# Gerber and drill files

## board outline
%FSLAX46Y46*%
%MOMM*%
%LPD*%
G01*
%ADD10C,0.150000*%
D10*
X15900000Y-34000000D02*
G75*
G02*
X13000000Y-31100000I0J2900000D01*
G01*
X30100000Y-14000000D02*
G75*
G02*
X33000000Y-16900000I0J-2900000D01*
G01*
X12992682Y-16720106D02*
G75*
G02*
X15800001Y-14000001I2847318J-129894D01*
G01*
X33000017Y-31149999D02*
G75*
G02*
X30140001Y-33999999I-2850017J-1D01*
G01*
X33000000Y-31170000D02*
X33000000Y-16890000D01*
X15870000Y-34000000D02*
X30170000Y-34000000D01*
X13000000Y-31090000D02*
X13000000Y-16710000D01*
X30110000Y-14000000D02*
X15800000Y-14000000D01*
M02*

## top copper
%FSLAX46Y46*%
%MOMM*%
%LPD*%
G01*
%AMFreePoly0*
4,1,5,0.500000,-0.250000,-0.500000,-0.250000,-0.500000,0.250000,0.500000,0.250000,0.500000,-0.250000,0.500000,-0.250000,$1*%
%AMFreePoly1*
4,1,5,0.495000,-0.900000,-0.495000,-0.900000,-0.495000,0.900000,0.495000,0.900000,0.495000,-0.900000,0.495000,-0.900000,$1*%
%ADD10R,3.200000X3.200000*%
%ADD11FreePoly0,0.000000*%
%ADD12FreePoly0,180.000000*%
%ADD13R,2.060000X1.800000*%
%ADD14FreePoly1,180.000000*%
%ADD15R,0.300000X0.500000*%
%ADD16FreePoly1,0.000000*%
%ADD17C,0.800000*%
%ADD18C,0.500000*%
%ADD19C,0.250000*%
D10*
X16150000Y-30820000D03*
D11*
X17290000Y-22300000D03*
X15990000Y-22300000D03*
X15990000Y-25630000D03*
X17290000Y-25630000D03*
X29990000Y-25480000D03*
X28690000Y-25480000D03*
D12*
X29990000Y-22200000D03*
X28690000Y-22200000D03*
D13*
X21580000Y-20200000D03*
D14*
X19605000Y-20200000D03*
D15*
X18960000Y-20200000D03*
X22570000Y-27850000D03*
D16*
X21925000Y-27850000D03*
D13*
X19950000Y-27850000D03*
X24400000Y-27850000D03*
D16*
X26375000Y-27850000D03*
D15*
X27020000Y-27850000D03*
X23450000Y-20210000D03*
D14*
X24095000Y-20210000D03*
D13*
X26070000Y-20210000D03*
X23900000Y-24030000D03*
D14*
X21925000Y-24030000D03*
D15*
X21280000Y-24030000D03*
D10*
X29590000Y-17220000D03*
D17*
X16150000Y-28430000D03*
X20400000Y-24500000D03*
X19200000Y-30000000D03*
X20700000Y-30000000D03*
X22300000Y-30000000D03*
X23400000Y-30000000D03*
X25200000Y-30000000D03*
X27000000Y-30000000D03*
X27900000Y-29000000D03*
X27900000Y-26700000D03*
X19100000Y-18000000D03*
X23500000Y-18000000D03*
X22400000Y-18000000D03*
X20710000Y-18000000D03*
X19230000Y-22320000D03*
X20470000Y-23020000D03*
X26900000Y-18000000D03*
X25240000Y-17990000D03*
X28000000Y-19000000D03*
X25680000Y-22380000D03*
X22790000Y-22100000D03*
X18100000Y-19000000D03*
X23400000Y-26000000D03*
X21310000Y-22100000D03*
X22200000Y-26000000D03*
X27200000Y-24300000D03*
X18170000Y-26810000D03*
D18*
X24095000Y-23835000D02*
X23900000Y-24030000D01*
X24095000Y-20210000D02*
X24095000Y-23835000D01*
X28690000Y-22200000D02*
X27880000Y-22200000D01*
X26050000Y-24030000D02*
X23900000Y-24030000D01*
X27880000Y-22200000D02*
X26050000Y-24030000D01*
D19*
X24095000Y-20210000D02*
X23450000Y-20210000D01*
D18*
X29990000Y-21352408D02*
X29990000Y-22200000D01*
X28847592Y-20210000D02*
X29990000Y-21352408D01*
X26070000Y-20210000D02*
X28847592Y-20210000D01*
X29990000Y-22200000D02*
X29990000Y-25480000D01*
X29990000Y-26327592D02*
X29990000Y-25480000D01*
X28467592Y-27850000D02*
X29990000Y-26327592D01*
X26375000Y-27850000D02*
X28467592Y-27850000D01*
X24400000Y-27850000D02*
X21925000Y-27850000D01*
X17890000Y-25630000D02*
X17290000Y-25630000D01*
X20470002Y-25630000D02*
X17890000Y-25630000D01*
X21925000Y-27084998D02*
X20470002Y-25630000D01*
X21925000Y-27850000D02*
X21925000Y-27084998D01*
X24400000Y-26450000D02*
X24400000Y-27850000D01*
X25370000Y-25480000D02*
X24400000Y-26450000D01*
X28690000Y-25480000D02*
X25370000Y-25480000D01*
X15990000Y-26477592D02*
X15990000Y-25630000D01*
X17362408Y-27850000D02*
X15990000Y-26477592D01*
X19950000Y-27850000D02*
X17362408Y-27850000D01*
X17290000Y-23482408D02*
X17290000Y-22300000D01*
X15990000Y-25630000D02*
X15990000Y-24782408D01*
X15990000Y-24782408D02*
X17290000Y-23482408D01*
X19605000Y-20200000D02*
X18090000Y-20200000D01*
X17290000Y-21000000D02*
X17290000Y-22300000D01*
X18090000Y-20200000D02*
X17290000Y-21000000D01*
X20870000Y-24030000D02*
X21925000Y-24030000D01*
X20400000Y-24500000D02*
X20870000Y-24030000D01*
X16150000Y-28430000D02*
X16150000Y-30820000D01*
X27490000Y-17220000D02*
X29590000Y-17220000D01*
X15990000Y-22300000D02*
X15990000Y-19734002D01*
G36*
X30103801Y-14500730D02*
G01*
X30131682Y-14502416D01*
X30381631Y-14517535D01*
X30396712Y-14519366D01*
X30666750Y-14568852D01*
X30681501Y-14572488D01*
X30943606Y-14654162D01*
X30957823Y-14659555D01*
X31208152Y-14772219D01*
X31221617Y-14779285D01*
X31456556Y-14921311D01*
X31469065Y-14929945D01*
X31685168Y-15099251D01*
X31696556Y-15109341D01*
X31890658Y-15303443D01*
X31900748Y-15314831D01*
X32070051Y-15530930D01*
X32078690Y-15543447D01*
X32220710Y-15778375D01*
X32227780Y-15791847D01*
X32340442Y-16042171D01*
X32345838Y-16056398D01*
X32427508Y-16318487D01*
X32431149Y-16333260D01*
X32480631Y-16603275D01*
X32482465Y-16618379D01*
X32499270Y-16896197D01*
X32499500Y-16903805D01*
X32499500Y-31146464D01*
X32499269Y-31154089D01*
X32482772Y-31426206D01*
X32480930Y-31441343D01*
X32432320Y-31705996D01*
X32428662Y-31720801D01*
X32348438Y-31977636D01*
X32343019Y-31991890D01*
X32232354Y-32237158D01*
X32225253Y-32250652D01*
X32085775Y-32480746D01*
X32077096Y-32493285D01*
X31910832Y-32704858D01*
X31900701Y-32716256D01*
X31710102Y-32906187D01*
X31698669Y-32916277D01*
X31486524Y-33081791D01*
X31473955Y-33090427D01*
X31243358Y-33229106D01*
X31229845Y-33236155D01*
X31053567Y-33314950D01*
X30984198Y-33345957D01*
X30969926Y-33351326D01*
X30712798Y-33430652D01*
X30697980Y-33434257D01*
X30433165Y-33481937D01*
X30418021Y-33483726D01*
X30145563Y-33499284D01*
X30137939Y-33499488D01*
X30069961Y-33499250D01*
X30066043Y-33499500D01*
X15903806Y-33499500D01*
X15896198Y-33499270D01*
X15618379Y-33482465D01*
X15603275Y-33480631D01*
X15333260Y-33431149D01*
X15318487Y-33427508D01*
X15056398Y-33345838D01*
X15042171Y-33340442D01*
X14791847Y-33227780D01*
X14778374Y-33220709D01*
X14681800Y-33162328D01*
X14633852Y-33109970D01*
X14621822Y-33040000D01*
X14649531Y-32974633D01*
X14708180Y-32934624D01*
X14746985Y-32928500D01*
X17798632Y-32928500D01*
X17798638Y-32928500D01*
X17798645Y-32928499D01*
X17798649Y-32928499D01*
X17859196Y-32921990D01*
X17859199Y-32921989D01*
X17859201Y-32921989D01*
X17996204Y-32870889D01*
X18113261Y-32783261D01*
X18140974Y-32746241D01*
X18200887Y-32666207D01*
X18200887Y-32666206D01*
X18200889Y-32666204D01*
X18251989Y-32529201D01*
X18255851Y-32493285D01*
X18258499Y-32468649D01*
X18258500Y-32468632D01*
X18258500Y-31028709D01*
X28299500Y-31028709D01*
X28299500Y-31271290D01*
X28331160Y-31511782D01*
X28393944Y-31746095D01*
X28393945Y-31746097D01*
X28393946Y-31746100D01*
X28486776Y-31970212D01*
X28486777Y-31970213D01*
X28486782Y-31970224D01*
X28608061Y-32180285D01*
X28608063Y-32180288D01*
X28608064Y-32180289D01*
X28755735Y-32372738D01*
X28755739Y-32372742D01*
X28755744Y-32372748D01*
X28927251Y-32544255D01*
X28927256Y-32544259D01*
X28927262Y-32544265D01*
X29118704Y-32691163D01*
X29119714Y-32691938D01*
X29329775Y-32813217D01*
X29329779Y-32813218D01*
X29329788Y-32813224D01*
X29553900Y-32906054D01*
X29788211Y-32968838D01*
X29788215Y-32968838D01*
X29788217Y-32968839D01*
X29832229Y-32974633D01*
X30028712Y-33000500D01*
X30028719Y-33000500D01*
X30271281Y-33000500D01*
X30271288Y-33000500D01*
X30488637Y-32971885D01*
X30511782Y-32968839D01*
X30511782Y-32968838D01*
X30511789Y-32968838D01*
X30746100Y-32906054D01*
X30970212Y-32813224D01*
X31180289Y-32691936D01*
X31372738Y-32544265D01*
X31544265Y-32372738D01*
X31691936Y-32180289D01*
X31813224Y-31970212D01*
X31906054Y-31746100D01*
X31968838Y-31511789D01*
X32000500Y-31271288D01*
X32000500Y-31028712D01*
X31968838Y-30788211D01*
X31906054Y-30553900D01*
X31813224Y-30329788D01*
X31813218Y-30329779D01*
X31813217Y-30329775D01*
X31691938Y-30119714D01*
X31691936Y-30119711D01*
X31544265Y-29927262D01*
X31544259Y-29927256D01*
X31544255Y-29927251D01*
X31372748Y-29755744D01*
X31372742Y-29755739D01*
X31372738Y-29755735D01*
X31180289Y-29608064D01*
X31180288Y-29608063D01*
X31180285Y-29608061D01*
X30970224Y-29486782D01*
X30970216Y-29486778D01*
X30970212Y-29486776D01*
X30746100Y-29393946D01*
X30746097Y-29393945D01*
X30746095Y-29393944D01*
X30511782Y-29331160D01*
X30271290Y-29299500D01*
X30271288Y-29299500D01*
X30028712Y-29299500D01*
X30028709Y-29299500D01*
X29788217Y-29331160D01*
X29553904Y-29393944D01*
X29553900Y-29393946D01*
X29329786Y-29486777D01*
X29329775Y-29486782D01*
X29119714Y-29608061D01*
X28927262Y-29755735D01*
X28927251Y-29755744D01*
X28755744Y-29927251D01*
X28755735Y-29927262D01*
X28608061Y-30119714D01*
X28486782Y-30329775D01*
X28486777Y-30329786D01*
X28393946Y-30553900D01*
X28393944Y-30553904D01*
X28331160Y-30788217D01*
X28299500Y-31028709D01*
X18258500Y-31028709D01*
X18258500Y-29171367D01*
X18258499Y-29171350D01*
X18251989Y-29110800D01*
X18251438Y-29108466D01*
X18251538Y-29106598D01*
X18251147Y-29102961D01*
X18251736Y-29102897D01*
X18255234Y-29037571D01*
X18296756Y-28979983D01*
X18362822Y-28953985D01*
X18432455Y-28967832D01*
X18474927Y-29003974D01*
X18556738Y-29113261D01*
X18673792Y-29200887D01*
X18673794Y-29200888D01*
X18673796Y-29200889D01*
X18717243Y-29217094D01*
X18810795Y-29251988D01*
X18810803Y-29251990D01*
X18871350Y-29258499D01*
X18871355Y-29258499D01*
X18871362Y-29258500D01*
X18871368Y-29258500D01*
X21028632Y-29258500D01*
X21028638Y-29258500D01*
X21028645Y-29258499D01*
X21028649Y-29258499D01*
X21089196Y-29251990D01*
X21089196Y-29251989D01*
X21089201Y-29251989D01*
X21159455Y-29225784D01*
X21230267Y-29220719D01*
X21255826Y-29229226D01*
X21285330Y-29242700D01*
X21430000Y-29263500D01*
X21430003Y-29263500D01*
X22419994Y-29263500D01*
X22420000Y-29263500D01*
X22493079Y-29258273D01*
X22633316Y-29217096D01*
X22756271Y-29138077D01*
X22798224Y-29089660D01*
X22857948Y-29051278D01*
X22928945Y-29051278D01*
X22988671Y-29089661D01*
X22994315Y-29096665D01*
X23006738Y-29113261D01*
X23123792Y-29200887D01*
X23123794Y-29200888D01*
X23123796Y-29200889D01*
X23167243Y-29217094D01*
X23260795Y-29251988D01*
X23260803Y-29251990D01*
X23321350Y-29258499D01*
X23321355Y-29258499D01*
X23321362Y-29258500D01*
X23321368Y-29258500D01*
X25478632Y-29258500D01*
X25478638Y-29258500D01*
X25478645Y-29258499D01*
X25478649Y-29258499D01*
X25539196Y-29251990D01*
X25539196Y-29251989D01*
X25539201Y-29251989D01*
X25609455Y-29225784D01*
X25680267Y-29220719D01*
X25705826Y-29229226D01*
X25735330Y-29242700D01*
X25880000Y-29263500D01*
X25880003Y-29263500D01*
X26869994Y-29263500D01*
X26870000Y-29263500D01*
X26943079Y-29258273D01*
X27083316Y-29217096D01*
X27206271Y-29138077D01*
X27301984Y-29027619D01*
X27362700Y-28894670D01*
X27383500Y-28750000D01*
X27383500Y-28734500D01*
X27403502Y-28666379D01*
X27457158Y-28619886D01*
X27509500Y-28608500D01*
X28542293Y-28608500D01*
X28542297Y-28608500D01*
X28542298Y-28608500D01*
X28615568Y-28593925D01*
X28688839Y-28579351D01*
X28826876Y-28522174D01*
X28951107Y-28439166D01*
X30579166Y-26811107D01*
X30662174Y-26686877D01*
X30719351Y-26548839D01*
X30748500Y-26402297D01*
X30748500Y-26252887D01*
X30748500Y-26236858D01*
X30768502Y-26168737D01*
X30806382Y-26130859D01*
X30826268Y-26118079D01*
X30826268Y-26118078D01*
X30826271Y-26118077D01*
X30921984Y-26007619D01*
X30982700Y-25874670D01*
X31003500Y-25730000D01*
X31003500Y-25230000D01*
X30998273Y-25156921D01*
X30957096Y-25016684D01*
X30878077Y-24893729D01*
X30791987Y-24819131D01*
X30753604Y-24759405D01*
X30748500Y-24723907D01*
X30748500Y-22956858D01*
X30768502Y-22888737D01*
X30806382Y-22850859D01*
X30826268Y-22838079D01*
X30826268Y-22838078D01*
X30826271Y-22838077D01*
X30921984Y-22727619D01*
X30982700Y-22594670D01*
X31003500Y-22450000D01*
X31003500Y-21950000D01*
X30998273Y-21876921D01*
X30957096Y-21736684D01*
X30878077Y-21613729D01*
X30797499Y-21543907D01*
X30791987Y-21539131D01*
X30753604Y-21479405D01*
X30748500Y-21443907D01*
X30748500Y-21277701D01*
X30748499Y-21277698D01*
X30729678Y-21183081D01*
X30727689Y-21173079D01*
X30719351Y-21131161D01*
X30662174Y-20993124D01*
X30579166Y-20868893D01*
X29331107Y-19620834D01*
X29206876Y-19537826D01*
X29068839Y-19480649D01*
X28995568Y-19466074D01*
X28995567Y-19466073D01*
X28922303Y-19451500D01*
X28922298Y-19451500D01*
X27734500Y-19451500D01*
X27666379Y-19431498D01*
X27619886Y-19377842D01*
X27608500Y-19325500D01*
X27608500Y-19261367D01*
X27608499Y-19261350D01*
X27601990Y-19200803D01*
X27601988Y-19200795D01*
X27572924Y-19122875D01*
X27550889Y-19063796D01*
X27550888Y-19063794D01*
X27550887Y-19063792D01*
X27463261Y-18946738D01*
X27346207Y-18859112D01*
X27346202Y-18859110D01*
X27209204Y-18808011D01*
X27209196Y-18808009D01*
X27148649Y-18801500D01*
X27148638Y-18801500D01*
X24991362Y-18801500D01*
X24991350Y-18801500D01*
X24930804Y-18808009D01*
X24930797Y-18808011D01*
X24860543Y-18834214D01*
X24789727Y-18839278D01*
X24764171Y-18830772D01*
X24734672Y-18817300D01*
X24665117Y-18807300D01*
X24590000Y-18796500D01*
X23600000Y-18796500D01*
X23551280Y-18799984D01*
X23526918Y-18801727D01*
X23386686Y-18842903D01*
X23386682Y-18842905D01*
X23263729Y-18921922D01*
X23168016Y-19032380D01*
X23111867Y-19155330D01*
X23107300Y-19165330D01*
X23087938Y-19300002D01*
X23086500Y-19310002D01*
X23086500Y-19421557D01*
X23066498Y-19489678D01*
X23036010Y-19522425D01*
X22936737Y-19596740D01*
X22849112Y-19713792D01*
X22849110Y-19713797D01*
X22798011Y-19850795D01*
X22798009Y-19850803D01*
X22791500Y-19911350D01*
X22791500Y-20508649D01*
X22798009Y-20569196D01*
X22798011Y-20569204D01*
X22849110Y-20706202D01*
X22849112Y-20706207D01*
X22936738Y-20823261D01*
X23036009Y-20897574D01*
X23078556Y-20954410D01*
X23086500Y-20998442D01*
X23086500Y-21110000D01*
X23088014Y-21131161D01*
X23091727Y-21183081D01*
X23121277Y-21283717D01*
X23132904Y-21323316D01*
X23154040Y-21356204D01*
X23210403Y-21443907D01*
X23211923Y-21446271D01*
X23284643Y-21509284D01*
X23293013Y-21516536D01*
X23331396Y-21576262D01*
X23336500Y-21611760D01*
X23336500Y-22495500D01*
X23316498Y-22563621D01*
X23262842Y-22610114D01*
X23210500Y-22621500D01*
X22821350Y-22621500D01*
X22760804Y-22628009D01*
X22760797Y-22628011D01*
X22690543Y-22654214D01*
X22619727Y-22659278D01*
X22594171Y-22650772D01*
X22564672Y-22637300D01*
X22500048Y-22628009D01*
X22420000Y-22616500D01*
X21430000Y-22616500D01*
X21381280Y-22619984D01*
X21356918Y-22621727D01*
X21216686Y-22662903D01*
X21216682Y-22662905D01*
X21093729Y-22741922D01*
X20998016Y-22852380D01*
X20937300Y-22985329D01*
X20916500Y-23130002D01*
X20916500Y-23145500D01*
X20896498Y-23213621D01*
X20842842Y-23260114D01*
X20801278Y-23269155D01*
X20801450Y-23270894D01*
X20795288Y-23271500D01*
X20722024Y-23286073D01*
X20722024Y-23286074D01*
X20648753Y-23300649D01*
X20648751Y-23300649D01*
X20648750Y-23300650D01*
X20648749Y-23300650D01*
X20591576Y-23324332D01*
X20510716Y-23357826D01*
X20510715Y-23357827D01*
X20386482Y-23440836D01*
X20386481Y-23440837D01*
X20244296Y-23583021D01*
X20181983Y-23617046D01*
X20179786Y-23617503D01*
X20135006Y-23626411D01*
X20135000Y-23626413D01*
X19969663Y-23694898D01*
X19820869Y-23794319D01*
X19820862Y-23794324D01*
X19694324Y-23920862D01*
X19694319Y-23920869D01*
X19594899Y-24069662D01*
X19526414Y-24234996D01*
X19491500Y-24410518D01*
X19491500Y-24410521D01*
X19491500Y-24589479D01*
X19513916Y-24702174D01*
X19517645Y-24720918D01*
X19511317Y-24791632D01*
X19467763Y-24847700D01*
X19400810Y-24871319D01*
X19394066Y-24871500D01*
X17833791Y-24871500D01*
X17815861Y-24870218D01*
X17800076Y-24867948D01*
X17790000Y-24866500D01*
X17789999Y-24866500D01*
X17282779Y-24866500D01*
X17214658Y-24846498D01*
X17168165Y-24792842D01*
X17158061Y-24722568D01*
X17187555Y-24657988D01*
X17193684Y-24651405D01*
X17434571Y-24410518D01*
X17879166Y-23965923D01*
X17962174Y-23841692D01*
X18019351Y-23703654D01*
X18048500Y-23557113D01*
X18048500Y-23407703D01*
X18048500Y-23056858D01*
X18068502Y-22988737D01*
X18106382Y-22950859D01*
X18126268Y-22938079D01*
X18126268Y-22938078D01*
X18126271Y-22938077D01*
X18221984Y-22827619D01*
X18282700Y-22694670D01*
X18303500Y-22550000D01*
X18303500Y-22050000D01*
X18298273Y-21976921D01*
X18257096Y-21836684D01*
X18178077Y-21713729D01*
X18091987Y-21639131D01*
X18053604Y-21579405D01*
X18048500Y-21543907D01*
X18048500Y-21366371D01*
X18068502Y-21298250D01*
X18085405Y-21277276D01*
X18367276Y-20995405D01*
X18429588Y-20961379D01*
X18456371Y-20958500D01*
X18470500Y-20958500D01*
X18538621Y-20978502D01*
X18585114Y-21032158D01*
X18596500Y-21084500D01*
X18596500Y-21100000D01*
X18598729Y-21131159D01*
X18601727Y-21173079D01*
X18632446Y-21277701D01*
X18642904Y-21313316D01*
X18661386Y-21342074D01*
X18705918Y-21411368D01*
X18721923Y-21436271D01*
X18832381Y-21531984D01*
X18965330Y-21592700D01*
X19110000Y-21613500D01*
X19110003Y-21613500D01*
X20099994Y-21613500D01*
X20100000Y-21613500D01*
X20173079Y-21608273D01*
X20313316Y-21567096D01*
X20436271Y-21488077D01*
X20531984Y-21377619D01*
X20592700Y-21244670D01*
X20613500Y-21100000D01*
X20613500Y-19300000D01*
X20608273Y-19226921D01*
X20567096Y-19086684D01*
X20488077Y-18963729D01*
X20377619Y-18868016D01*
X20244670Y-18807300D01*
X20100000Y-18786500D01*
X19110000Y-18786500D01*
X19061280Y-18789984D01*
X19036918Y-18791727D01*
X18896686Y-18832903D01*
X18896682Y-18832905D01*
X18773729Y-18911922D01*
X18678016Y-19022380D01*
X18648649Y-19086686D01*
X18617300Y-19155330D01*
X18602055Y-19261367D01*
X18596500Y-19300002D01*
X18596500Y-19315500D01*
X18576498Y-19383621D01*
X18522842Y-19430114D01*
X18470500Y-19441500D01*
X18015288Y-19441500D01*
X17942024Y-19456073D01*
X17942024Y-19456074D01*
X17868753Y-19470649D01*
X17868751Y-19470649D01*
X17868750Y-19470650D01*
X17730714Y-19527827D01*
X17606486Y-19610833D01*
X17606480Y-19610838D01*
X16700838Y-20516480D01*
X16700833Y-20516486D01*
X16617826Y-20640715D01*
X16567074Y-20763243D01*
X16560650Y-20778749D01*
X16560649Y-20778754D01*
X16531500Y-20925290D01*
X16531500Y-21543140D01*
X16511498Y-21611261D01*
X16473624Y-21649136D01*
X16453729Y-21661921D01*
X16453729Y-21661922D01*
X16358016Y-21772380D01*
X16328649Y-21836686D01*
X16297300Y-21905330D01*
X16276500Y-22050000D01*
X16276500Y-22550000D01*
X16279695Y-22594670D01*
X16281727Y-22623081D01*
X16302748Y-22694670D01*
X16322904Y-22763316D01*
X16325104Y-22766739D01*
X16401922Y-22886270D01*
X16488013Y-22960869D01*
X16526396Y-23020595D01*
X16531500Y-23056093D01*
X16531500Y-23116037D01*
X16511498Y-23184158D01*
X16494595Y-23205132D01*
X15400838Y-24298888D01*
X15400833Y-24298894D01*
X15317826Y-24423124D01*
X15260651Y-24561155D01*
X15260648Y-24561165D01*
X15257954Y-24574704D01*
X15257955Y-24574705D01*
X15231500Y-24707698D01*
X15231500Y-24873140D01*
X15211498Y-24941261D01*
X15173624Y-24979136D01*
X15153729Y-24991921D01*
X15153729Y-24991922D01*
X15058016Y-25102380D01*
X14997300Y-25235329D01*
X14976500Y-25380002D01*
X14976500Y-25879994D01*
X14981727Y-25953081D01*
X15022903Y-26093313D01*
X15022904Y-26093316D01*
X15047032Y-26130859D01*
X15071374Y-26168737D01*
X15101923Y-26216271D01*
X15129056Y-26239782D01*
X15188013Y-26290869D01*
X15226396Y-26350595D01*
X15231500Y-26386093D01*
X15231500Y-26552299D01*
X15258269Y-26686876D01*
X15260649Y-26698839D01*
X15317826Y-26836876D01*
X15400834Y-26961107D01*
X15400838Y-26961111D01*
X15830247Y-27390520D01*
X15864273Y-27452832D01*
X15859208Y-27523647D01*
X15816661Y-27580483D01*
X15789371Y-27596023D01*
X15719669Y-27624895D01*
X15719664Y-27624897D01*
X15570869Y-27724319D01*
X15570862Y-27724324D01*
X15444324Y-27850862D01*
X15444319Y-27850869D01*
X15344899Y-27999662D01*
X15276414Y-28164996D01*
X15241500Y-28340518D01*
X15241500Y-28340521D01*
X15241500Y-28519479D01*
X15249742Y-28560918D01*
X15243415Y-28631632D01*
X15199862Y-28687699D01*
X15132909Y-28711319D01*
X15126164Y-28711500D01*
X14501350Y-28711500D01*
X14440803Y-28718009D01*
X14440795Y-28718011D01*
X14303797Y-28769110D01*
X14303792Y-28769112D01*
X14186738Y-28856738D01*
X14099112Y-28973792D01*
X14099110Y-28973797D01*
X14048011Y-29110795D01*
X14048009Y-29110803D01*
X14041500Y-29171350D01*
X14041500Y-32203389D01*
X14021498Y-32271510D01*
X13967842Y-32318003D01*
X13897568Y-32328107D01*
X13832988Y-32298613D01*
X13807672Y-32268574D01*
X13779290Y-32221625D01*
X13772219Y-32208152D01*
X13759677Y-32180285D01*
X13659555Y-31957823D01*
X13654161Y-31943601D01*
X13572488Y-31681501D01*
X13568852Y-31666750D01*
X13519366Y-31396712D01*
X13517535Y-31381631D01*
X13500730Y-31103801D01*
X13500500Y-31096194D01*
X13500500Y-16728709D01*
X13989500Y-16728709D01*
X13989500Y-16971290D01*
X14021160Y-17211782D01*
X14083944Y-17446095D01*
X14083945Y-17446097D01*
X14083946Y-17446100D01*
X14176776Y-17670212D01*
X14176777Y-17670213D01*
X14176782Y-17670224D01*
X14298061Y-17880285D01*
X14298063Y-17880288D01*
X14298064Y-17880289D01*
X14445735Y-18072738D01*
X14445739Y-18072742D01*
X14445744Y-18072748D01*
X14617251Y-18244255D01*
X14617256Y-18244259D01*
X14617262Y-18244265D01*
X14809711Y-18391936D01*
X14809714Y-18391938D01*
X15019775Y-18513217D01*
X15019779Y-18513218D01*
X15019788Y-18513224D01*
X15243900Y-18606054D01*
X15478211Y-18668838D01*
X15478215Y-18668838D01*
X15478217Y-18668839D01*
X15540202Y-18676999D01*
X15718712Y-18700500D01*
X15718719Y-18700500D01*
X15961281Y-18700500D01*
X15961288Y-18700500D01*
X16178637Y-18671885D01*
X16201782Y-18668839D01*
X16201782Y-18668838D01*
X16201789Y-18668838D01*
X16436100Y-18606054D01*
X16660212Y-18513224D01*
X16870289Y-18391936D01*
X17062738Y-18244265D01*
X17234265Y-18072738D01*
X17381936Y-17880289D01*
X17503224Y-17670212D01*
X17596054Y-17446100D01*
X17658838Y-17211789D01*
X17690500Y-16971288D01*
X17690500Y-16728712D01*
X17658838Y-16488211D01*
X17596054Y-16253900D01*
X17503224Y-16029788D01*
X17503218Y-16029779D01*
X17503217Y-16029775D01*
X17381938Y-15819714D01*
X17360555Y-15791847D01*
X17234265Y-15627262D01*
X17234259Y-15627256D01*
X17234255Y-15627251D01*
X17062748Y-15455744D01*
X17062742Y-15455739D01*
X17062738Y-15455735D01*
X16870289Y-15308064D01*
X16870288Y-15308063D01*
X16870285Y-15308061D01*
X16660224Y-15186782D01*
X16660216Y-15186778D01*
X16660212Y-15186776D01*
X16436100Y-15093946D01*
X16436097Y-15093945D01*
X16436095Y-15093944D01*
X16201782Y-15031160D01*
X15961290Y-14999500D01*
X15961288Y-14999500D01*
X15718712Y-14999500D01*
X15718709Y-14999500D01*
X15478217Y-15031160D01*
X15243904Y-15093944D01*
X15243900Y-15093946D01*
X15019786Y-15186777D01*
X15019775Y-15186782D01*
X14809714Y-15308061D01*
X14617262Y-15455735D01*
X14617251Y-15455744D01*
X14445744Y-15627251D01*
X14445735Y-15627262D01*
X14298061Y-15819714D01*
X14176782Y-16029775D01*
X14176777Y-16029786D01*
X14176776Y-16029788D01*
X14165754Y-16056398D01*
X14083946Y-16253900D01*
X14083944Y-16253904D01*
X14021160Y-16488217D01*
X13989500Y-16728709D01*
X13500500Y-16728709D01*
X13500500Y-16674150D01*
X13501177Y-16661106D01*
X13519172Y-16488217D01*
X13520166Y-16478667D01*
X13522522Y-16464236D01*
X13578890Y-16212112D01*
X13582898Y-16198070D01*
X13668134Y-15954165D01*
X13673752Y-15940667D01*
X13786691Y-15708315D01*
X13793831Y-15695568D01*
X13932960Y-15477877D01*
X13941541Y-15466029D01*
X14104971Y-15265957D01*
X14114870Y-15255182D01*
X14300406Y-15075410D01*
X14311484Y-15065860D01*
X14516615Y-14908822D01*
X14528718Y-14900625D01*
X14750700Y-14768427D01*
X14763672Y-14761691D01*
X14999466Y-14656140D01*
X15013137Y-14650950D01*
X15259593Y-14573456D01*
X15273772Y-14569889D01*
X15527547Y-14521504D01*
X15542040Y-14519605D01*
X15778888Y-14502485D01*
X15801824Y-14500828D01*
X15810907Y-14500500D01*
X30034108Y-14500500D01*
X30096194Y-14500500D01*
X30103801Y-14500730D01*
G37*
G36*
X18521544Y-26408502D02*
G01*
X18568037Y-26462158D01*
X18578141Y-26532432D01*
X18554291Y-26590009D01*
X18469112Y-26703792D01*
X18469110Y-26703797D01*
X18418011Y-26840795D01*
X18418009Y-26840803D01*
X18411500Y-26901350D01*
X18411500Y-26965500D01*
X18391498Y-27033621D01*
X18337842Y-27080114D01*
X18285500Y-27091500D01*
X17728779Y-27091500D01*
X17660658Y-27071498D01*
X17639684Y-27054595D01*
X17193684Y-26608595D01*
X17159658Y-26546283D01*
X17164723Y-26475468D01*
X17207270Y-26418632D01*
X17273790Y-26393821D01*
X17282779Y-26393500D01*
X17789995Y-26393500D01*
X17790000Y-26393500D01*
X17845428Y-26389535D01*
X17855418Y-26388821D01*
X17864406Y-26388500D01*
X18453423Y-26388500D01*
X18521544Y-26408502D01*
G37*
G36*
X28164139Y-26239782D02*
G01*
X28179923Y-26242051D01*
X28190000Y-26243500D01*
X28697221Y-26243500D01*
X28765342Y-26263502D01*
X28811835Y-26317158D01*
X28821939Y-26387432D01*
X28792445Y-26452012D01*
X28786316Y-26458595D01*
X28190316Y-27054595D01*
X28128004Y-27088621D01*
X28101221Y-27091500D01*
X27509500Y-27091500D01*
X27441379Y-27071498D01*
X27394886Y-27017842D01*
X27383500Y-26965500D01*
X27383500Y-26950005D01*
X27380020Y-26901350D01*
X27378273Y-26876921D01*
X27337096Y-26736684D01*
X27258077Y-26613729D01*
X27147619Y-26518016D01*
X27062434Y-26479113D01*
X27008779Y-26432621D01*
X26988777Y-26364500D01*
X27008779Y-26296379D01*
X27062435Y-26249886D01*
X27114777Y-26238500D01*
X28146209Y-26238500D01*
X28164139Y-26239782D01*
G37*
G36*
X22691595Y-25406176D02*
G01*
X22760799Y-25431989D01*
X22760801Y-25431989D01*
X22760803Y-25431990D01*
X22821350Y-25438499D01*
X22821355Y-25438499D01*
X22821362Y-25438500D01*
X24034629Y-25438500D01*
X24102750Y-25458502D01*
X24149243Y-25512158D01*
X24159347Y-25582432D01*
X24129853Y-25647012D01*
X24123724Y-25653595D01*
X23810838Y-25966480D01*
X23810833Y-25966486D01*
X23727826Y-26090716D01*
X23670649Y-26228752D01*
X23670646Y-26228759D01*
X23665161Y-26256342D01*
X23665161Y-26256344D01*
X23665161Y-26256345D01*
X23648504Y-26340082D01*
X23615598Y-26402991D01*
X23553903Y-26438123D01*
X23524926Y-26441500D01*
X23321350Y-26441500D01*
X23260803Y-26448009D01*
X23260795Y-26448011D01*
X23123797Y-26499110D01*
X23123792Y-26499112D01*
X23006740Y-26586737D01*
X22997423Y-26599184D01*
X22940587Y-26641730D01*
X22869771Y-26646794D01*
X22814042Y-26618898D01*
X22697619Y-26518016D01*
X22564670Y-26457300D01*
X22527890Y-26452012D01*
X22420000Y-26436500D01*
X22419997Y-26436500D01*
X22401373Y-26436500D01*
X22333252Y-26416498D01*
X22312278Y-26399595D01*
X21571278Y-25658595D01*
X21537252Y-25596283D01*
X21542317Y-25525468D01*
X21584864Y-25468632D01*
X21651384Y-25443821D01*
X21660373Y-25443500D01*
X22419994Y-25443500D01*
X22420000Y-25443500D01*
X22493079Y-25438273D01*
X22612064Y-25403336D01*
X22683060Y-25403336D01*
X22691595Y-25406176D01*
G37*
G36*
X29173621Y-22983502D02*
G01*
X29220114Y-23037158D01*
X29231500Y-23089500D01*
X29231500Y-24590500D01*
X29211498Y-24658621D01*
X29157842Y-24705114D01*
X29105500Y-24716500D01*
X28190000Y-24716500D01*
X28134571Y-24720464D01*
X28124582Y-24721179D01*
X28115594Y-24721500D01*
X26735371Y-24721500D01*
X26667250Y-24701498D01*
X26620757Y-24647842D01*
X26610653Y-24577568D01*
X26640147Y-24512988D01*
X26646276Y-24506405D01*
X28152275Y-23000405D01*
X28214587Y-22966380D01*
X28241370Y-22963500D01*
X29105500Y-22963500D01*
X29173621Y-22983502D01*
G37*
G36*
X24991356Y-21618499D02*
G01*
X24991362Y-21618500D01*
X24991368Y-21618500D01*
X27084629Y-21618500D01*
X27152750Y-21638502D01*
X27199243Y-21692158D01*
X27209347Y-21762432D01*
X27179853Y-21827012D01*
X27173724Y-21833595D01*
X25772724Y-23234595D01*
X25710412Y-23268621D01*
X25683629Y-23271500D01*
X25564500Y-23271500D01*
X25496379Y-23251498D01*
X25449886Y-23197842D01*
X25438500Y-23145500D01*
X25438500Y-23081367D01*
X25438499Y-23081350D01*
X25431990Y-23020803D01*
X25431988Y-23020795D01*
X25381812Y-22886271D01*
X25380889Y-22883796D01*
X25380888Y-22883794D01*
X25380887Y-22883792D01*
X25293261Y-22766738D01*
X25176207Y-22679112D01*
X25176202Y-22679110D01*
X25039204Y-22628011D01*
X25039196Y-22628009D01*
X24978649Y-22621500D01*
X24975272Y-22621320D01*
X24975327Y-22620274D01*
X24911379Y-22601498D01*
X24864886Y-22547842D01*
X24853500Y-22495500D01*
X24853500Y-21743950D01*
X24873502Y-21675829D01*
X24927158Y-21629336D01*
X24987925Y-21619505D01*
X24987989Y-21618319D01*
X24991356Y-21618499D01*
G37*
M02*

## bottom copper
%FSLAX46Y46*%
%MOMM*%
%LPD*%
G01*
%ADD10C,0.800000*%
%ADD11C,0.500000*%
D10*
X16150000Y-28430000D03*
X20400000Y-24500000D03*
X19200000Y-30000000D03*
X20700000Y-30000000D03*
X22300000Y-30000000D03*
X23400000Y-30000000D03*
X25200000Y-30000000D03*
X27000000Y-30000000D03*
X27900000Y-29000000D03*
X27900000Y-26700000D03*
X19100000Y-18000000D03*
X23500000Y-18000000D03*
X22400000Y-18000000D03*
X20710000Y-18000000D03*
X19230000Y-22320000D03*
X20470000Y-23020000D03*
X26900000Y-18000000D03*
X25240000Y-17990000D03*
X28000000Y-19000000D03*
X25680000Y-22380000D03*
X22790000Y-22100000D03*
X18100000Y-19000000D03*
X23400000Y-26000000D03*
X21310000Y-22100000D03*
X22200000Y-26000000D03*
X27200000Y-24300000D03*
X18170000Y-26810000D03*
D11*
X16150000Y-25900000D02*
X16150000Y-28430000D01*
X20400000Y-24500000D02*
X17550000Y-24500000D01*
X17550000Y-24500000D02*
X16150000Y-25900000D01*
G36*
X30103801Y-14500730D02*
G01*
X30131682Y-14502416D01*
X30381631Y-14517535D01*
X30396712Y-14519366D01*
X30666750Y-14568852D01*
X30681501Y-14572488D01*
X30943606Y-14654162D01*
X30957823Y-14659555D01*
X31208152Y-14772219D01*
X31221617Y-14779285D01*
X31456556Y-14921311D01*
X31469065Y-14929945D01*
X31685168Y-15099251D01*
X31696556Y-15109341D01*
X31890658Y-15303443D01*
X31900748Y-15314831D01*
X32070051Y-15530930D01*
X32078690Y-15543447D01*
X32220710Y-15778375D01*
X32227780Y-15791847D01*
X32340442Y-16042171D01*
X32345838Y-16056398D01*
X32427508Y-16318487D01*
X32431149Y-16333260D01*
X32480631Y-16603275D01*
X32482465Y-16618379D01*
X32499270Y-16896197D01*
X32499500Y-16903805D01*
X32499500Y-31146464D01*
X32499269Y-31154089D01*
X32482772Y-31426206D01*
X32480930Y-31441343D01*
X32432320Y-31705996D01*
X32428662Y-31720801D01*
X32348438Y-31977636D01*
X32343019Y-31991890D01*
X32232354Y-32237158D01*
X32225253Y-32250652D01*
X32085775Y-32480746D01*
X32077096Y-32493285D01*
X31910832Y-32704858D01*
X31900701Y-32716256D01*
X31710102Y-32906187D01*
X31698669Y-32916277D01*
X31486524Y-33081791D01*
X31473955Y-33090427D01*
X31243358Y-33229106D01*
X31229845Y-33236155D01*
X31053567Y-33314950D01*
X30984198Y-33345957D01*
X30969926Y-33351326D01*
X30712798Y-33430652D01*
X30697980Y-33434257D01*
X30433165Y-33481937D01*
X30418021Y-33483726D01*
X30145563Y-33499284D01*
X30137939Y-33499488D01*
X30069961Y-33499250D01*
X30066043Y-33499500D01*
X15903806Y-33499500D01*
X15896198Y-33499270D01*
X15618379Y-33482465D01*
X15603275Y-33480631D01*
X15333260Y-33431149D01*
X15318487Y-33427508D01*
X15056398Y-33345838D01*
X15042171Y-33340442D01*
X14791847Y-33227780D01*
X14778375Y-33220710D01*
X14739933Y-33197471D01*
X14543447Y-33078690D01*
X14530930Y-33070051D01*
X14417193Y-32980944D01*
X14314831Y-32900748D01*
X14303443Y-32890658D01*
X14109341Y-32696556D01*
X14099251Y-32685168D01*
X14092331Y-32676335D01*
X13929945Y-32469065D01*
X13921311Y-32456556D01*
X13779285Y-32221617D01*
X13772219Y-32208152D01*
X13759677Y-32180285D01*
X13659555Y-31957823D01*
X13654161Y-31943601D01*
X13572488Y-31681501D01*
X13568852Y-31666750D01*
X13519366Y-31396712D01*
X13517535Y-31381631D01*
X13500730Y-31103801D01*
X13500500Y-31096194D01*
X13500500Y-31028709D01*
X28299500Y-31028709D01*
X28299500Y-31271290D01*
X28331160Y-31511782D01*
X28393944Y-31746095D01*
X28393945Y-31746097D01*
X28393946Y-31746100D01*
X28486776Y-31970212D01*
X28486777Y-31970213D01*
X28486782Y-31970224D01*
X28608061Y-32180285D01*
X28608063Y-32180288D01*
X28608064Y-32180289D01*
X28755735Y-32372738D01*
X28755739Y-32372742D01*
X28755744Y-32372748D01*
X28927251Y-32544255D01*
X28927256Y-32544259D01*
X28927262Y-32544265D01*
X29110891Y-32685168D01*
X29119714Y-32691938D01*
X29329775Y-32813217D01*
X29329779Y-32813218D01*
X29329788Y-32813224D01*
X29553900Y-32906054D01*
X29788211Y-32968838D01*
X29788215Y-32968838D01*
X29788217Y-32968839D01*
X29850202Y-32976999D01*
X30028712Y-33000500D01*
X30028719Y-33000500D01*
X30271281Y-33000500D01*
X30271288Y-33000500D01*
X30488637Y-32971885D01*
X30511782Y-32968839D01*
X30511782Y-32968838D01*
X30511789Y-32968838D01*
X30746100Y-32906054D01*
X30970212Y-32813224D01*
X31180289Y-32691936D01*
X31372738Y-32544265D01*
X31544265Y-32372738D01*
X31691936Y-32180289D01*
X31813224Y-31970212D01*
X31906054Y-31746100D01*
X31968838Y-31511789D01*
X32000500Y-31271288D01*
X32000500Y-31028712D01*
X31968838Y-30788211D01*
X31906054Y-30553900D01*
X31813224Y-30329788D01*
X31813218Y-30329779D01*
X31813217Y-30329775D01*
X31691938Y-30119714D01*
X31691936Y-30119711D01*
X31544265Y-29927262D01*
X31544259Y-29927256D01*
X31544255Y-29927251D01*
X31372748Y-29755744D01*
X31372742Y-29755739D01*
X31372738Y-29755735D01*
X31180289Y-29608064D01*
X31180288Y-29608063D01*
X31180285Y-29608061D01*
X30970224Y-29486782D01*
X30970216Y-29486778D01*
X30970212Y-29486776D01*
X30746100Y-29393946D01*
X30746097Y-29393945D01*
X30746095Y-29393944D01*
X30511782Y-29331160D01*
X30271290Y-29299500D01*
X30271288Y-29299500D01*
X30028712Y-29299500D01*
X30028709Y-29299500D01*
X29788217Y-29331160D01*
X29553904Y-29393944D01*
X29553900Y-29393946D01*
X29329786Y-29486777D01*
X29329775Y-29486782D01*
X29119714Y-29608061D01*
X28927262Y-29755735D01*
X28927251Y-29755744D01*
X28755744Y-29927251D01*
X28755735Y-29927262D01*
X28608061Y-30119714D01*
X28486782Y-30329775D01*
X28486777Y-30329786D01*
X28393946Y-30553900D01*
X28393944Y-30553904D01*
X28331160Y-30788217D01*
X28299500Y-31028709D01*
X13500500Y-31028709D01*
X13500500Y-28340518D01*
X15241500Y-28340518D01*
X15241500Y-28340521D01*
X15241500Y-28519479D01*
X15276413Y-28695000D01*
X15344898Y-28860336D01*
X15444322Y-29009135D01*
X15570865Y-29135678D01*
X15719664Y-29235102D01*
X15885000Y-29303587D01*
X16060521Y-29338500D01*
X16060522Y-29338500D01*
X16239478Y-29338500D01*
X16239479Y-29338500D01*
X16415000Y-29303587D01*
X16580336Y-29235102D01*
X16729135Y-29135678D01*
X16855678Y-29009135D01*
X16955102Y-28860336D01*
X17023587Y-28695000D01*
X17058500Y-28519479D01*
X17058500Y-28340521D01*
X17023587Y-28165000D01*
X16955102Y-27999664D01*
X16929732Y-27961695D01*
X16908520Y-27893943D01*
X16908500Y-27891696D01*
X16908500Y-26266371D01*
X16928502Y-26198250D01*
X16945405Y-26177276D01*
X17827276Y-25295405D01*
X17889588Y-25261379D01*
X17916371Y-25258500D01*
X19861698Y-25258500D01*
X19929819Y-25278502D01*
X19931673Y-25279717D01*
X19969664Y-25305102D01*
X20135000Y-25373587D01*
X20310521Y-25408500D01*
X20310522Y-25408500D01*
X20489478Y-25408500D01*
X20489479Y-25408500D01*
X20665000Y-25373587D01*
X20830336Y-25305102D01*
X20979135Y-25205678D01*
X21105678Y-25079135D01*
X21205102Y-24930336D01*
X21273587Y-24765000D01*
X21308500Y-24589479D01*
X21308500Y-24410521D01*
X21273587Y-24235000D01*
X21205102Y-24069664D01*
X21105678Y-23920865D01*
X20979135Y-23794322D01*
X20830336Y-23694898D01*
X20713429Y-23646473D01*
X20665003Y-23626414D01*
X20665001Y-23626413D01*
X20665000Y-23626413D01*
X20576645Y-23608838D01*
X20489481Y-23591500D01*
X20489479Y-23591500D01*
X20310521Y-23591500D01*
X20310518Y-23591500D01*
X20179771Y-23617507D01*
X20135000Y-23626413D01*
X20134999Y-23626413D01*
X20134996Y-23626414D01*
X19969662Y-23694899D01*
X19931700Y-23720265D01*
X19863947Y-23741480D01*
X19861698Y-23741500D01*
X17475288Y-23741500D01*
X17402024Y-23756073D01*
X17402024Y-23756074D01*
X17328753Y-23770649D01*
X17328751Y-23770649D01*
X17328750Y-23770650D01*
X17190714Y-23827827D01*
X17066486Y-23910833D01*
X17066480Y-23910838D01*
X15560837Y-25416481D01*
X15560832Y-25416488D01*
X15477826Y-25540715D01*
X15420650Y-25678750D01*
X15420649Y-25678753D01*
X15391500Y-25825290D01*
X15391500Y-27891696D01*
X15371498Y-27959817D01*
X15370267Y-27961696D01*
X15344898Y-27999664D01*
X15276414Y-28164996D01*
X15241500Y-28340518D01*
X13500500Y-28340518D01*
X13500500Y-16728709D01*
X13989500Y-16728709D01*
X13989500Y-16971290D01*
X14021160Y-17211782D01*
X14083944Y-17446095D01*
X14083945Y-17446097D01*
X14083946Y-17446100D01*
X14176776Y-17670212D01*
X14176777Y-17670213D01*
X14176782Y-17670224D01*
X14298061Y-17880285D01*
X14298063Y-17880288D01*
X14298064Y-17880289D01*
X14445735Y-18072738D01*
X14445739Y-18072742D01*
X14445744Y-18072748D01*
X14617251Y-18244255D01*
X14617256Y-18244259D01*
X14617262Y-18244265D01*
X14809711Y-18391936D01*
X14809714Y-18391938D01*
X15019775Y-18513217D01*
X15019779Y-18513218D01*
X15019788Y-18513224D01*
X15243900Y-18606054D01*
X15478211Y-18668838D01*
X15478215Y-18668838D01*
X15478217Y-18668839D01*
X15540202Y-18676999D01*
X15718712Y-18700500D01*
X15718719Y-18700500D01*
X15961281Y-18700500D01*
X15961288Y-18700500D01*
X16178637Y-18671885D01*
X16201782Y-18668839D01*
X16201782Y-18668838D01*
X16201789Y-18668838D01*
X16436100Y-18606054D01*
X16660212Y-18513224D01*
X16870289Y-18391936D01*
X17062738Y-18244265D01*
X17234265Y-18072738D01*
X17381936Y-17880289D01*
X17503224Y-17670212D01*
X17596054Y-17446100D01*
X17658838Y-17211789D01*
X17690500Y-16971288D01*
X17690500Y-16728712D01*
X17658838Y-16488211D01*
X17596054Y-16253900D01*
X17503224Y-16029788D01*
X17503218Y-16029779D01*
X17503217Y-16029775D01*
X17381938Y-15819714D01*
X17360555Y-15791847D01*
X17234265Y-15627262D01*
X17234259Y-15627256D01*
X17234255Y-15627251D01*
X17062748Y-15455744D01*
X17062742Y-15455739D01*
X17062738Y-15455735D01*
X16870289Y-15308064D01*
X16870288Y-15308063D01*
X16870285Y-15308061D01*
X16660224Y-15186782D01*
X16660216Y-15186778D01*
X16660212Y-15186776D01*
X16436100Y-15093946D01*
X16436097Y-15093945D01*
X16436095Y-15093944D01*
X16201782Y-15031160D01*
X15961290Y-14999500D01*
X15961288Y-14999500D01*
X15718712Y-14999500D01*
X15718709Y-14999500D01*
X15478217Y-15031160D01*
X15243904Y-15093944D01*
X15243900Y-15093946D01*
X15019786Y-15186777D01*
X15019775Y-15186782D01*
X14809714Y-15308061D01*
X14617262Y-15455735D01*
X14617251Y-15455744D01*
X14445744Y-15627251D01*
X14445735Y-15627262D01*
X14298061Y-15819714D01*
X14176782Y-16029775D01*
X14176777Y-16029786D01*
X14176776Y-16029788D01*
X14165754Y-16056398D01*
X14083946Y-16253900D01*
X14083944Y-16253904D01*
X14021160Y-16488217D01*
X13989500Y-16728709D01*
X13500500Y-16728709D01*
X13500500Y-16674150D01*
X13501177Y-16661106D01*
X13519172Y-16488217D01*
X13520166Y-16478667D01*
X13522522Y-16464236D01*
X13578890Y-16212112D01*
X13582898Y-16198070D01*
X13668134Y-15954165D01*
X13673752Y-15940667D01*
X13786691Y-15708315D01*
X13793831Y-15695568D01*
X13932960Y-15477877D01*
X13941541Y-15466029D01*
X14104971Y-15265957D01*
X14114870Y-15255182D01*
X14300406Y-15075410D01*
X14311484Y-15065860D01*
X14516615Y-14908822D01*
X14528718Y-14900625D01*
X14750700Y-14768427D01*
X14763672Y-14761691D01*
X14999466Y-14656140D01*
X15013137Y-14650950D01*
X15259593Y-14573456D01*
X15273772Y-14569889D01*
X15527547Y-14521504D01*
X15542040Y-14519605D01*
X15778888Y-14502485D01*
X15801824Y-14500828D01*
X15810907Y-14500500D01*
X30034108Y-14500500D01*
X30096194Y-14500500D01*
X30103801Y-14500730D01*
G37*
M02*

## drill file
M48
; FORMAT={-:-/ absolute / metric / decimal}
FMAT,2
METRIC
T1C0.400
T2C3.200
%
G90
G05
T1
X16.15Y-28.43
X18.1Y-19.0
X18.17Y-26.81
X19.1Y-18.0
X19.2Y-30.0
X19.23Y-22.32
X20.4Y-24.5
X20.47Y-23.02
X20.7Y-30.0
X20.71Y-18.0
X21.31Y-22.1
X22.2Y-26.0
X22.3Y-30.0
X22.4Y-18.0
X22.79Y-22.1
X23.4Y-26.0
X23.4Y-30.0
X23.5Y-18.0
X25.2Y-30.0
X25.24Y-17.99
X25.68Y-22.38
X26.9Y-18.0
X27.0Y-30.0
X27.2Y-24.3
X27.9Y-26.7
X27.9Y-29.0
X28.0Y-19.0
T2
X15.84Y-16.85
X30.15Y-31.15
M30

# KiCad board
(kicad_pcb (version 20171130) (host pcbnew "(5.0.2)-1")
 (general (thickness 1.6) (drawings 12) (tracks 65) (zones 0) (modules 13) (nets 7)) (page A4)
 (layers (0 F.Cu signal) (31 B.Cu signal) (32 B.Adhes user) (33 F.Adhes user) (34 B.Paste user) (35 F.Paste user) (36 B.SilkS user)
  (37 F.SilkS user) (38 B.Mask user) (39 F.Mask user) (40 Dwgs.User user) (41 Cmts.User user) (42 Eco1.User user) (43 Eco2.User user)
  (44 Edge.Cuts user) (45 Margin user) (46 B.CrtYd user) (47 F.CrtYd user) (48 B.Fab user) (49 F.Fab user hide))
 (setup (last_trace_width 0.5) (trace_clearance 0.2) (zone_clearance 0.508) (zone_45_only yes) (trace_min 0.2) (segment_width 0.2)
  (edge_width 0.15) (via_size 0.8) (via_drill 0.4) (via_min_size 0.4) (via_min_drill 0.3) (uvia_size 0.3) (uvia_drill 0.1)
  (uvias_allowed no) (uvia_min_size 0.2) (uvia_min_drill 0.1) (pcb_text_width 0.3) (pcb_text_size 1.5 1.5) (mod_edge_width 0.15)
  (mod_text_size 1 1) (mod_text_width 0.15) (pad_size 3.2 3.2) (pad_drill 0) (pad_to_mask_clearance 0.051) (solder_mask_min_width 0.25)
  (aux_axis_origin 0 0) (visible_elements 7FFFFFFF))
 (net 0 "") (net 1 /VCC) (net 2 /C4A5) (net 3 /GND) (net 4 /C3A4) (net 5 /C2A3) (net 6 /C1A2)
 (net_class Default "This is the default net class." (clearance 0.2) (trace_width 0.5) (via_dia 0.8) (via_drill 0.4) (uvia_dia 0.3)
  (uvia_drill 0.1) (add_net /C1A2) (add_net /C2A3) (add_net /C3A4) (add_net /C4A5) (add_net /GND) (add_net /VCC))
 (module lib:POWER (layer F.Cu) (at 16.15 30.82) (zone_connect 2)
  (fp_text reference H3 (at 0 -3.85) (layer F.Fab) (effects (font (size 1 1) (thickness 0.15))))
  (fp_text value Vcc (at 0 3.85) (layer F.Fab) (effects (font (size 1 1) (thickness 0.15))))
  (pad 1 smd rect (at 0 0) (size 3.2 3.2) (layers F.Cu F.Paste F.Mask) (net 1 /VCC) (zone_connect 2)))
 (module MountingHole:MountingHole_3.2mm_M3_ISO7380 (layer F.Cu) (at 30.15 31.15)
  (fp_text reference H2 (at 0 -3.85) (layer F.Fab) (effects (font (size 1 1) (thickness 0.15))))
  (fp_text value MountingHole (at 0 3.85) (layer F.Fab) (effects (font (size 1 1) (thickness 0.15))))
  (pad 1 np_thru_hole circle (at 0 0) (size 3.2 3.2) (drill 3.2) (layers *.Cu *.Mask)))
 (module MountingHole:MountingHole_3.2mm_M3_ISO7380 (layer F.Cu) (at 15.84 16.85)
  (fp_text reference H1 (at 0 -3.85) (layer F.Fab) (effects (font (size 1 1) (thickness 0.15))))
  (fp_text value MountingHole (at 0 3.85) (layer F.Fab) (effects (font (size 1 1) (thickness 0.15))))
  (pad 1 np_thru_hole circle (at 0 0) (size 3.2 3.2) (drill 3.2) (layers *.Cu *.Mask)))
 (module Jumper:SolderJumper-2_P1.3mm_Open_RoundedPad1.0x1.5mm (layer F.Cu) (at 16.64 22.3)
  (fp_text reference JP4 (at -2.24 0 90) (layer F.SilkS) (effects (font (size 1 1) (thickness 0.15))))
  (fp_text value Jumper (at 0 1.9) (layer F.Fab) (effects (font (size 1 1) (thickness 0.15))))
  (pad 2 smd custom (at 0.65 0) (size 1 0.5) (layers F.Cu F.Mask) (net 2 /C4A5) (zone_connect 2) (options (clearance outline) (anchor rect))
   (primitives))
  (pad 1 smd custom (at -0.65 0) (size 1 0.5) (layers F.Cu F.Mask) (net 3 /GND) (zone_connect 2) (options (clearance outline) (anchor rect))
   (primitives)))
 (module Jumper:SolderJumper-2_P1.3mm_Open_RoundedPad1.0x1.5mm (layer F.Cu) (at 16.64 25.63)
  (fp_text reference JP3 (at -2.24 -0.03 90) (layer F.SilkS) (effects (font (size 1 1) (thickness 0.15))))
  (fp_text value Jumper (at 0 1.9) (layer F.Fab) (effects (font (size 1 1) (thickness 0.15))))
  (pad 1 smd custom (at -0.65 0) (size 1 0.5) (layers F.Cu F.Mask) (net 2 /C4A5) (zone_connect 2)
   (options (clearance outline) (anchor rect)) (primitives))
  (pad 2 smd custom (at 0.65 0) (size 1 0.5) (layers F.Cu F.Mask) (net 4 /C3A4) (zone_connect 2) (options (clearance outline) (anchor rect))
   (primitives)))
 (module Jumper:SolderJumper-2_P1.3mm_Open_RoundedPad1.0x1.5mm (layer F.Cu) (at 29.34 25.48)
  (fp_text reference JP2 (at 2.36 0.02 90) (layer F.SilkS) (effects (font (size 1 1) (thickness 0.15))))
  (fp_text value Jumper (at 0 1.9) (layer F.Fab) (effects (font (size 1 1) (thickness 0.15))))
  (pad 2 smd custom (at 0.65 0) (size 1 0.5) (layers F.Cu F.Mask) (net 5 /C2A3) (zone_connect 2) (options (clearance outline) (anchor rect))
   (primitives))
  (pad 1 smd custom (at -0.65 0) (size 1 0.5) (layers F.Cu F.Mask) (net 4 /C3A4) (zone_connect 2)
   (options (clearance outline) (anchor rect)) (primitives)))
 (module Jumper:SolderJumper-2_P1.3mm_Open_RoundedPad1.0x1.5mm (layer F.Cu) (at 29.34 22.2 180)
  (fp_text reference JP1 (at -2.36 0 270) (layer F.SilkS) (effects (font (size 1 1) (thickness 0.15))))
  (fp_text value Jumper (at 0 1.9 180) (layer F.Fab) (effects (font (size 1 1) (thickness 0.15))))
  (pad 1 smd custom (at -0.65 0 180) (size 1 0.5) (layers F.Cu F.Mask) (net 5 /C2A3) (zone_connect 2)
   (options (clearance outline) (anchor rect)) (primitives))
  (pad 2 smd custom (at 0.65 0 180) (size 1 0.5) (layers F.Cu F.Mask) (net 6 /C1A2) (zone_connect 2)
   (options (clearance outline) (anchor rect)) (primitives)))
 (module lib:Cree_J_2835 (layer F.Cu) (at 21.58 20.2 180)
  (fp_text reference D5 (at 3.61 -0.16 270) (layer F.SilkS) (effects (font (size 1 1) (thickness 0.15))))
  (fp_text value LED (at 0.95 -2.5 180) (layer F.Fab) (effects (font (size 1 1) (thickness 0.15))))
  (pad 1 smd rect (at 0 0 180) (size 2.06 1.8) (layers F.Cu F.Paste F.Mask) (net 3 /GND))
  (pad 2 smd custom (at 1.975 0 180) (size 0.99 1.8) (layers F.Cu F.Paste F.Mask) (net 2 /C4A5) (zone_connect 0)
   (options (clearance outline) (anchor rect)) (primitives))
  (pad 2 smd rect (at 2.62 0 180) (size 0.3 0.5) (layers F.Cu F.Paste F.Mask) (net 2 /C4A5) (zone_connect 0)))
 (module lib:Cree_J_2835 (layer F.Cu) (at 19.95 27.85)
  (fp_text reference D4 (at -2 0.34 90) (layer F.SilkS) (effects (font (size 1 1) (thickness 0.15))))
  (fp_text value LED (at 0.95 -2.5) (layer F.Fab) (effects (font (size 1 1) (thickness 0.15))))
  (pad 2 smd rect (at 2.62 0) (size 0.3 0.5) (layers F.Cu F.Paste F.Mask) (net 4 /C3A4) (zone_connect 0))
  (pad 2 smd custom (at 1.975 0) (size 0.99 1.8) (layers F.Cu F.Paste F.Mask) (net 4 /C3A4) (zone_connect 0)
   (options (clearance outline) (anchor rect)) (primitives))
  (pad 1 smd rect (at 0 0) (size 2.06 1.8) (layers F.Cu F.Paste F.Mask) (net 2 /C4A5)))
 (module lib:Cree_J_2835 (layer F.Cu) (at 24.4 27.85)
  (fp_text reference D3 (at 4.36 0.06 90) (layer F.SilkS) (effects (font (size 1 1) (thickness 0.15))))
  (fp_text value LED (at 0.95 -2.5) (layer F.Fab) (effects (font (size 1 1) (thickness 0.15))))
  (pad 1 smd rect (at 0 0) (size 2.06 1.8) (layers F.Cu F.Paste F.Mask) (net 4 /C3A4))
  (pad 2 smd custom (at 1.975 0) (size 0.99 1.8) (layers F.Cu F.Paste F.Mask) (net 5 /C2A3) (zone_connect 0)
   (options (clearance outline) (anchor rect)) (primitives))
  (pad 2 smd rect (at 2.62 0) (size 0.3 0.5) (layers F.Cu F.Paste F.Mask) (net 5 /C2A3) (zone_connect 0)))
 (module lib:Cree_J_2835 (layer F.Cu) (at 26.07 20.21 180)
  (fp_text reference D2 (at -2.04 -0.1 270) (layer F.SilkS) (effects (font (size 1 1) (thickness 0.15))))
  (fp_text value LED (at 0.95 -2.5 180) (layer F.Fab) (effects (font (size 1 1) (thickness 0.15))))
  (pad 2 smd rect (at 2.62 0 180) (size 0.3 0.5) (layers F.Cu F.Paste F.Mask) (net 6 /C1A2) (zone_connect 0))
  (pad 2 smd custom (at 1.975 0 180) (size 0.99 1.8) (layers F.Cu F.Paste F.Mask) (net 6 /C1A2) (zone_connect 0)
   (options (clearance outline) (anchor rect)) (primitives))
  (pad 1 smd rect (at 0 0 180) (size 2.06 1.8) (layers F.Cu F.Paste F.Mask) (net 5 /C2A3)))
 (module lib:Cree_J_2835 (layer F.Cu) (at 23.9 24.03 180)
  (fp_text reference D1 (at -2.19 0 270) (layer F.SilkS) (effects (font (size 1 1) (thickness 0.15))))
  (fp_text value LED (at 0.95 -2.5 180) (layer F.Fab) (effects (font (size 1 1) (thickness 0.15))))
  (pad 1 smd rect (at 0 0 180) (size 2.06 1.8) (layers F.Cu F.Paste F.Mask) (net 6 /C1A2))
  (pad 2 smd custom (at 1.975 0 180) (size 0.99 1.8) (layers F.Cu F.Paste F.Mask) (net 1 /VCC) (zone_connect 0)
   (options (clearance outline) (anchor rect)) (primitives))
  (pad 2 smd rect (at 2.62 0 180) (size 0.3 0.5) (layers F.Cu F.Paste F.Mask) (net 1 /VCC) (zone_connect 0)))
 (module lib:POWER (layer F.Cu) (at 29.59 17.22) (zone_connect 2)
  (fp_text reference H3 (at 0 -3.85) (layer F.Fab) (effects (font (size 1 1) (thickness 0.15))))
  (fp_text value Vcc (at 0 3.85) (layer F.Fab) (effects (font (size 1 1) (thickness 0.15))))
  (pad 1 smd rect (at 0 0) (size 3.2 3.2) (layers F.Cu F.Paste F.Mask) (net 3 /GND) (zone_connect 2)))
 (gr_arc (start 15.9 31.1) (end 13 31.1) (angle -90) (layer Edge.Cuts) (width 0.15))
 (gr_arc (start 30.1 16.9) (end 33 16.9) (angle -90) (layer Edge.Cuts) (width 0.15))
 (gr_arc (start 15.84 16.85) (end 15.800001 14.000001) (angle -86.58391779) (layer Edge.Cuts) (width 0.15))
 (gr_arc (start 30.15 31.15) (end 30.140001 33.999999) (angle -90.201037) (layer Edge.Cuts) (width 0.15))
 (gr_line (start 33 31.17) (end 33 16.89) (layer Edge.Cuts) (width 0.15))
 (gr_line (start 15.87 34) (end 30.17 34) (layer Edge.Cuts) (width 0.15))
 (gr_line (start 13 31.09) (end 13 16.71) (layer Edge.Cuts) (width 0.15))
 (gr_line (start 30.11 14) (end 15.8 14) (layer Edge.Cuts) (width 0.15))
 (segment (start 24.095 23.835) (end 23.9 24.03) (width 0.5) (layer F.Cu) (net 6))
 (segment (start 24.095 20.21) (end 24.095 23.835) (width 0.5) (layer F.Cu) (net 6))
 (segment (start 28.69 22.2) (end 27.88 22.2) (width 0.5) (layer F.Cu) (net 6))
 (segment (start 26.05 24.03) (end 23.9 24.03) (width 0.5) (layer F.Cu) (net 6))
 (segment (start 27.88 22.2) (end 26.05 24.03) (width 0.5) (layer F.Cu) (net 6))
 (segment (start 24.095 20.21) (end 23.45 20.21) (width 0.25) (layer F.Cu) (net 6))
 (segment (start 29.99 21.352408) (end 29.99 22.2) (width 0.5) (layer F.Cu) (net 5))
 (segment (start 28.847592 20.21) (end 29.99 21.352408) (width 0.5) (layer F.Cu) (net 5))
 (segment (start 26.07 20.21) (end 28.847592 20.21) (width 0.5) (layer F.Cu) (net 5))
 (segment (start 29.99 22.2) (end 29.99 25.48) (width 0.5) (layer F.Cu) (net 5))
 (segment (start 29.99 26.327592) (end 29.99 25.48) (width 0.5) (layer F.Cu) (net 5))
 (segment (start 28.467592 27.85) (end 29.99 26.327592) (width 0.5) (layer F.Cu) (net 5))
 (segment (start 26.375 27.85) (end 28.467592 27.85) (width 0.5) (layer F.Cu) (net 5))
 (segment (start 24.4 27.85) (end 21.925 27.85) (width 0.5) (layer F.Cu) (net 4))
 (segment (start 17.89 25.63) (end 17.29 25.63) (width 0.5) (layer F.Cu) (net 4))
 (segment (start 20.470002 25.63) (end 17.89 25.63) (width 0.5) (layer F.Cu) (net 4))
 (segment (start 21.925 27.084998) (end 20.470002 25.63) (width 0.5) (layer F.Cu) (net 4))
 (segment (start 21.925 27.85) (end 21.925 27.084998) (width 0.5) (layer F.Cu) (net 4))
 (segment (start 24.4 26.45) (end 24.4 27.85) (width 0.5) (layer F.Cu) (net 4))
 (segment (start 25.37 25.48) (end 24.4 26.45) (width 0.5) (layer F.Cu) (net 4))
 (segment (start 28.69 25.48) (end 25.37 25.48) (width 0.5) (layer F.Cu) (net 4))
 (segment (start 15.99 26.477592) (end 15.99 25.63) (width 0.5) (layer F.Cu) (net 2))
 (segment (start 17.362408 27.85) (end 15.99 26.477592) (width 0.5) (layer F.Cu) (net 2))
 (segment (start 19.95 27.85) (end 17.362408 27.85) (width 0.5) (layer F.Cu) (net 2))
 (segment (start 17.29 23.482408) (end 17.29 22.3) (width 0.5) (layer F.Cu) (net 2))
 (segment (start 15.99 25.63) (end 15.99 24.782408) (width 0.5) (layer F.Cu) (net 2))
 (segment (start 15.99 24.782408) (end 17.29 23.482408) (width 0.5) (layer F.Cu) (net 2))
 (segment (start 19.605 20.2) (end 18.09 20.2) (width 0.5) (layer F.Cu) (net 2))
 (segment (start 17.29 21) (end 17.29 22.3) (width 0.5) (layer F.Cu) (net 2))
 (segment (start 18.09 20.2) (end 17.29 21) (width 0.5) (layer F.Cu) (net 2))
 (via (at 16.15 28.43) (size 0.8) (drill 0.4) (layers F.Cu B.Cu) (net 1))
 (segment (start 20.87 24.03) (end 21.925 24.03) (width 0.5) (layer F.Cu) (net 1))
 (segment (start 20.4 24.5) (end 20.87 24.03) (width 0.5) (layer F.Cu) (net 1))
 (segment (start 16.15 28.43) (end 16.15 30.82) (width 0.5) (layer F.Cu) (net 1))
 (via (at 20.4 24.5) (size 0.8) (drill 0.4) (layers F.Cu B.Cu) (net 1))
 (segment (start 16.15 25.9) (end 16.15 28.43) (width 0.5) (layer B.Cu) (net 1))
 (segment (start 20.4 24.5) (end 17.55 24.5) (width 0.5) (layer B.Cu) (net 1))
 (segment (start 17.55 24.5) (end 16.15 25.9) (width 0.5) (layer B.Cu) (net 1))
 (segment (start 27.49 17.22) (end 29.59 17.22) (width 0.5) (layer F.Cu) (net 3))
 (segment (start 15.99 22.3) (end 15.99 19.734002) (width 0.5) (layer F.Cu) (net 3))
 (via (at 19.2 30) (size 0.8) (drill 0.4) (layers F.Cu B.Cu) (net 3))
 (via (at 20.7 30) (size 0.8) (drill 0.4) (layers F.Cu B.Cu) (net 3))
 (via (at 22.3 30) (size 0.8) (drill 0.4) (layers F.Cu B.Cu) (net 3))
 (via (at 23.4 30) (size 0.8) (drill 0.4) (layers F.Cu B.Cu) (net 3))
 (via (at 25.2 30) (size 0.8) (drill 0.4) (layers F.Cu B.Cu) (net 3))
 (via (at 27 30) (size 0.8) (drill 0.4) (layers F.Cu B.Cu) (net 3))
 (via (at 27.9 29) (size 0.8) (drill 0.4) (layers F.Cu B.Cu) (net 3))
 (via (at 27.9 26.7) (size 0.8) (drill 0.4) (layers F.Cu B.Cu) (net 3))
 (via (at 19.1 18) (size 0.8) (drill 0.4) (layers F.Cu B.Cu) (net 3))
 (via (at 23.5 18) (size 0.8) (drill 0.4) (layers F.Cu B.Cu) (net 3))
 (via (at 22.4 18) (size 0.8) (drill 0.4) (layers F.Cu B.Cu) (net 3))
 (via (at 20.71 18) (size 0.8) (drill 0.4) (layers F.Cu B.Cu) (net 3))
 (via (at 19.23 22.32) (size 0.8) (drill 0.4) (layers F.Cu B.Cu) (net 3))
 (via (at 20.47 23.02) (size 0.8) (drill 0.4) (layers F.Cu B.Cu) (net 3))
 (via (at 26.9 18) (size 0.8) (drill 0.4) (layers F.Cu B.Cu) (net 3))
 (via (at 25.24 17.99) (size 0.8) (drill 0.4) (layers F.Cu B.Cu) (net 3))
 (via (at 28 19) (size 0.8) (drill 0.4) (layers F.Cu B.Cu) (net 3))
 (via (at 25.68 22.38) (size 0.8) (drill 0.4) (layers F.Cu B.Cu) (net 3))
 (via (at 22.79 22.1) (size 0.8) (drill 0.4) (layers F.Cu B.Cu) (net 3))
 (via (at 18.1 19) (size 0.8) (drill 0.4) (layers F.Cu B.Cu) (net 3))
 (via (at 23.4 26) (size 0.8) (drill 0.4) (layers F.Cu B.Cu) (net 3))
 (via (at 21.31 22.1) (size 0.8) (drill 0.4) (layers F.Cu B.Cu) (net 3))
 (via (at 22.2 26) (size 0.8) (drill 0.4) (layers F.Cu B.Cu) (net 3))
 (via (at 27.2 24.3) (size 0.8) (drill 0.4) (layers F.Cu B.Cu) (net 3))
 (via (at 18.17 26.81) (size 0.8) (drill 0.4) (layers F.Cu B.Cu) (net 3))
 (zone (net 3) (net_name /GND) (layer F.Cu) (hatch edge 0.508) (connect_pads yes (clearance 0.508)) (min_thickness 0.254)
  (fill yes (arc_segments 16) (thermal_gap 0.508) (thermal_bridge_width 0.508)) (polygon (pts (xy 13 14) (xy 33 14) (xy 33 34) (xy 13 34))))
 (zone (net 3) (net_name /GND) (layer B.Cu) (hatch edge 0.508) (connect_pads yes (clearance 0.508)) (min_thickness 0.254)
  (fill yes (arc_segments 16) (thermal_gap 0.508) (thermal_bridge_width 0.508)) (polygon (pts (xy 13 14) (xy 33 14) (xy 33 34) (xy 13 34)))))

